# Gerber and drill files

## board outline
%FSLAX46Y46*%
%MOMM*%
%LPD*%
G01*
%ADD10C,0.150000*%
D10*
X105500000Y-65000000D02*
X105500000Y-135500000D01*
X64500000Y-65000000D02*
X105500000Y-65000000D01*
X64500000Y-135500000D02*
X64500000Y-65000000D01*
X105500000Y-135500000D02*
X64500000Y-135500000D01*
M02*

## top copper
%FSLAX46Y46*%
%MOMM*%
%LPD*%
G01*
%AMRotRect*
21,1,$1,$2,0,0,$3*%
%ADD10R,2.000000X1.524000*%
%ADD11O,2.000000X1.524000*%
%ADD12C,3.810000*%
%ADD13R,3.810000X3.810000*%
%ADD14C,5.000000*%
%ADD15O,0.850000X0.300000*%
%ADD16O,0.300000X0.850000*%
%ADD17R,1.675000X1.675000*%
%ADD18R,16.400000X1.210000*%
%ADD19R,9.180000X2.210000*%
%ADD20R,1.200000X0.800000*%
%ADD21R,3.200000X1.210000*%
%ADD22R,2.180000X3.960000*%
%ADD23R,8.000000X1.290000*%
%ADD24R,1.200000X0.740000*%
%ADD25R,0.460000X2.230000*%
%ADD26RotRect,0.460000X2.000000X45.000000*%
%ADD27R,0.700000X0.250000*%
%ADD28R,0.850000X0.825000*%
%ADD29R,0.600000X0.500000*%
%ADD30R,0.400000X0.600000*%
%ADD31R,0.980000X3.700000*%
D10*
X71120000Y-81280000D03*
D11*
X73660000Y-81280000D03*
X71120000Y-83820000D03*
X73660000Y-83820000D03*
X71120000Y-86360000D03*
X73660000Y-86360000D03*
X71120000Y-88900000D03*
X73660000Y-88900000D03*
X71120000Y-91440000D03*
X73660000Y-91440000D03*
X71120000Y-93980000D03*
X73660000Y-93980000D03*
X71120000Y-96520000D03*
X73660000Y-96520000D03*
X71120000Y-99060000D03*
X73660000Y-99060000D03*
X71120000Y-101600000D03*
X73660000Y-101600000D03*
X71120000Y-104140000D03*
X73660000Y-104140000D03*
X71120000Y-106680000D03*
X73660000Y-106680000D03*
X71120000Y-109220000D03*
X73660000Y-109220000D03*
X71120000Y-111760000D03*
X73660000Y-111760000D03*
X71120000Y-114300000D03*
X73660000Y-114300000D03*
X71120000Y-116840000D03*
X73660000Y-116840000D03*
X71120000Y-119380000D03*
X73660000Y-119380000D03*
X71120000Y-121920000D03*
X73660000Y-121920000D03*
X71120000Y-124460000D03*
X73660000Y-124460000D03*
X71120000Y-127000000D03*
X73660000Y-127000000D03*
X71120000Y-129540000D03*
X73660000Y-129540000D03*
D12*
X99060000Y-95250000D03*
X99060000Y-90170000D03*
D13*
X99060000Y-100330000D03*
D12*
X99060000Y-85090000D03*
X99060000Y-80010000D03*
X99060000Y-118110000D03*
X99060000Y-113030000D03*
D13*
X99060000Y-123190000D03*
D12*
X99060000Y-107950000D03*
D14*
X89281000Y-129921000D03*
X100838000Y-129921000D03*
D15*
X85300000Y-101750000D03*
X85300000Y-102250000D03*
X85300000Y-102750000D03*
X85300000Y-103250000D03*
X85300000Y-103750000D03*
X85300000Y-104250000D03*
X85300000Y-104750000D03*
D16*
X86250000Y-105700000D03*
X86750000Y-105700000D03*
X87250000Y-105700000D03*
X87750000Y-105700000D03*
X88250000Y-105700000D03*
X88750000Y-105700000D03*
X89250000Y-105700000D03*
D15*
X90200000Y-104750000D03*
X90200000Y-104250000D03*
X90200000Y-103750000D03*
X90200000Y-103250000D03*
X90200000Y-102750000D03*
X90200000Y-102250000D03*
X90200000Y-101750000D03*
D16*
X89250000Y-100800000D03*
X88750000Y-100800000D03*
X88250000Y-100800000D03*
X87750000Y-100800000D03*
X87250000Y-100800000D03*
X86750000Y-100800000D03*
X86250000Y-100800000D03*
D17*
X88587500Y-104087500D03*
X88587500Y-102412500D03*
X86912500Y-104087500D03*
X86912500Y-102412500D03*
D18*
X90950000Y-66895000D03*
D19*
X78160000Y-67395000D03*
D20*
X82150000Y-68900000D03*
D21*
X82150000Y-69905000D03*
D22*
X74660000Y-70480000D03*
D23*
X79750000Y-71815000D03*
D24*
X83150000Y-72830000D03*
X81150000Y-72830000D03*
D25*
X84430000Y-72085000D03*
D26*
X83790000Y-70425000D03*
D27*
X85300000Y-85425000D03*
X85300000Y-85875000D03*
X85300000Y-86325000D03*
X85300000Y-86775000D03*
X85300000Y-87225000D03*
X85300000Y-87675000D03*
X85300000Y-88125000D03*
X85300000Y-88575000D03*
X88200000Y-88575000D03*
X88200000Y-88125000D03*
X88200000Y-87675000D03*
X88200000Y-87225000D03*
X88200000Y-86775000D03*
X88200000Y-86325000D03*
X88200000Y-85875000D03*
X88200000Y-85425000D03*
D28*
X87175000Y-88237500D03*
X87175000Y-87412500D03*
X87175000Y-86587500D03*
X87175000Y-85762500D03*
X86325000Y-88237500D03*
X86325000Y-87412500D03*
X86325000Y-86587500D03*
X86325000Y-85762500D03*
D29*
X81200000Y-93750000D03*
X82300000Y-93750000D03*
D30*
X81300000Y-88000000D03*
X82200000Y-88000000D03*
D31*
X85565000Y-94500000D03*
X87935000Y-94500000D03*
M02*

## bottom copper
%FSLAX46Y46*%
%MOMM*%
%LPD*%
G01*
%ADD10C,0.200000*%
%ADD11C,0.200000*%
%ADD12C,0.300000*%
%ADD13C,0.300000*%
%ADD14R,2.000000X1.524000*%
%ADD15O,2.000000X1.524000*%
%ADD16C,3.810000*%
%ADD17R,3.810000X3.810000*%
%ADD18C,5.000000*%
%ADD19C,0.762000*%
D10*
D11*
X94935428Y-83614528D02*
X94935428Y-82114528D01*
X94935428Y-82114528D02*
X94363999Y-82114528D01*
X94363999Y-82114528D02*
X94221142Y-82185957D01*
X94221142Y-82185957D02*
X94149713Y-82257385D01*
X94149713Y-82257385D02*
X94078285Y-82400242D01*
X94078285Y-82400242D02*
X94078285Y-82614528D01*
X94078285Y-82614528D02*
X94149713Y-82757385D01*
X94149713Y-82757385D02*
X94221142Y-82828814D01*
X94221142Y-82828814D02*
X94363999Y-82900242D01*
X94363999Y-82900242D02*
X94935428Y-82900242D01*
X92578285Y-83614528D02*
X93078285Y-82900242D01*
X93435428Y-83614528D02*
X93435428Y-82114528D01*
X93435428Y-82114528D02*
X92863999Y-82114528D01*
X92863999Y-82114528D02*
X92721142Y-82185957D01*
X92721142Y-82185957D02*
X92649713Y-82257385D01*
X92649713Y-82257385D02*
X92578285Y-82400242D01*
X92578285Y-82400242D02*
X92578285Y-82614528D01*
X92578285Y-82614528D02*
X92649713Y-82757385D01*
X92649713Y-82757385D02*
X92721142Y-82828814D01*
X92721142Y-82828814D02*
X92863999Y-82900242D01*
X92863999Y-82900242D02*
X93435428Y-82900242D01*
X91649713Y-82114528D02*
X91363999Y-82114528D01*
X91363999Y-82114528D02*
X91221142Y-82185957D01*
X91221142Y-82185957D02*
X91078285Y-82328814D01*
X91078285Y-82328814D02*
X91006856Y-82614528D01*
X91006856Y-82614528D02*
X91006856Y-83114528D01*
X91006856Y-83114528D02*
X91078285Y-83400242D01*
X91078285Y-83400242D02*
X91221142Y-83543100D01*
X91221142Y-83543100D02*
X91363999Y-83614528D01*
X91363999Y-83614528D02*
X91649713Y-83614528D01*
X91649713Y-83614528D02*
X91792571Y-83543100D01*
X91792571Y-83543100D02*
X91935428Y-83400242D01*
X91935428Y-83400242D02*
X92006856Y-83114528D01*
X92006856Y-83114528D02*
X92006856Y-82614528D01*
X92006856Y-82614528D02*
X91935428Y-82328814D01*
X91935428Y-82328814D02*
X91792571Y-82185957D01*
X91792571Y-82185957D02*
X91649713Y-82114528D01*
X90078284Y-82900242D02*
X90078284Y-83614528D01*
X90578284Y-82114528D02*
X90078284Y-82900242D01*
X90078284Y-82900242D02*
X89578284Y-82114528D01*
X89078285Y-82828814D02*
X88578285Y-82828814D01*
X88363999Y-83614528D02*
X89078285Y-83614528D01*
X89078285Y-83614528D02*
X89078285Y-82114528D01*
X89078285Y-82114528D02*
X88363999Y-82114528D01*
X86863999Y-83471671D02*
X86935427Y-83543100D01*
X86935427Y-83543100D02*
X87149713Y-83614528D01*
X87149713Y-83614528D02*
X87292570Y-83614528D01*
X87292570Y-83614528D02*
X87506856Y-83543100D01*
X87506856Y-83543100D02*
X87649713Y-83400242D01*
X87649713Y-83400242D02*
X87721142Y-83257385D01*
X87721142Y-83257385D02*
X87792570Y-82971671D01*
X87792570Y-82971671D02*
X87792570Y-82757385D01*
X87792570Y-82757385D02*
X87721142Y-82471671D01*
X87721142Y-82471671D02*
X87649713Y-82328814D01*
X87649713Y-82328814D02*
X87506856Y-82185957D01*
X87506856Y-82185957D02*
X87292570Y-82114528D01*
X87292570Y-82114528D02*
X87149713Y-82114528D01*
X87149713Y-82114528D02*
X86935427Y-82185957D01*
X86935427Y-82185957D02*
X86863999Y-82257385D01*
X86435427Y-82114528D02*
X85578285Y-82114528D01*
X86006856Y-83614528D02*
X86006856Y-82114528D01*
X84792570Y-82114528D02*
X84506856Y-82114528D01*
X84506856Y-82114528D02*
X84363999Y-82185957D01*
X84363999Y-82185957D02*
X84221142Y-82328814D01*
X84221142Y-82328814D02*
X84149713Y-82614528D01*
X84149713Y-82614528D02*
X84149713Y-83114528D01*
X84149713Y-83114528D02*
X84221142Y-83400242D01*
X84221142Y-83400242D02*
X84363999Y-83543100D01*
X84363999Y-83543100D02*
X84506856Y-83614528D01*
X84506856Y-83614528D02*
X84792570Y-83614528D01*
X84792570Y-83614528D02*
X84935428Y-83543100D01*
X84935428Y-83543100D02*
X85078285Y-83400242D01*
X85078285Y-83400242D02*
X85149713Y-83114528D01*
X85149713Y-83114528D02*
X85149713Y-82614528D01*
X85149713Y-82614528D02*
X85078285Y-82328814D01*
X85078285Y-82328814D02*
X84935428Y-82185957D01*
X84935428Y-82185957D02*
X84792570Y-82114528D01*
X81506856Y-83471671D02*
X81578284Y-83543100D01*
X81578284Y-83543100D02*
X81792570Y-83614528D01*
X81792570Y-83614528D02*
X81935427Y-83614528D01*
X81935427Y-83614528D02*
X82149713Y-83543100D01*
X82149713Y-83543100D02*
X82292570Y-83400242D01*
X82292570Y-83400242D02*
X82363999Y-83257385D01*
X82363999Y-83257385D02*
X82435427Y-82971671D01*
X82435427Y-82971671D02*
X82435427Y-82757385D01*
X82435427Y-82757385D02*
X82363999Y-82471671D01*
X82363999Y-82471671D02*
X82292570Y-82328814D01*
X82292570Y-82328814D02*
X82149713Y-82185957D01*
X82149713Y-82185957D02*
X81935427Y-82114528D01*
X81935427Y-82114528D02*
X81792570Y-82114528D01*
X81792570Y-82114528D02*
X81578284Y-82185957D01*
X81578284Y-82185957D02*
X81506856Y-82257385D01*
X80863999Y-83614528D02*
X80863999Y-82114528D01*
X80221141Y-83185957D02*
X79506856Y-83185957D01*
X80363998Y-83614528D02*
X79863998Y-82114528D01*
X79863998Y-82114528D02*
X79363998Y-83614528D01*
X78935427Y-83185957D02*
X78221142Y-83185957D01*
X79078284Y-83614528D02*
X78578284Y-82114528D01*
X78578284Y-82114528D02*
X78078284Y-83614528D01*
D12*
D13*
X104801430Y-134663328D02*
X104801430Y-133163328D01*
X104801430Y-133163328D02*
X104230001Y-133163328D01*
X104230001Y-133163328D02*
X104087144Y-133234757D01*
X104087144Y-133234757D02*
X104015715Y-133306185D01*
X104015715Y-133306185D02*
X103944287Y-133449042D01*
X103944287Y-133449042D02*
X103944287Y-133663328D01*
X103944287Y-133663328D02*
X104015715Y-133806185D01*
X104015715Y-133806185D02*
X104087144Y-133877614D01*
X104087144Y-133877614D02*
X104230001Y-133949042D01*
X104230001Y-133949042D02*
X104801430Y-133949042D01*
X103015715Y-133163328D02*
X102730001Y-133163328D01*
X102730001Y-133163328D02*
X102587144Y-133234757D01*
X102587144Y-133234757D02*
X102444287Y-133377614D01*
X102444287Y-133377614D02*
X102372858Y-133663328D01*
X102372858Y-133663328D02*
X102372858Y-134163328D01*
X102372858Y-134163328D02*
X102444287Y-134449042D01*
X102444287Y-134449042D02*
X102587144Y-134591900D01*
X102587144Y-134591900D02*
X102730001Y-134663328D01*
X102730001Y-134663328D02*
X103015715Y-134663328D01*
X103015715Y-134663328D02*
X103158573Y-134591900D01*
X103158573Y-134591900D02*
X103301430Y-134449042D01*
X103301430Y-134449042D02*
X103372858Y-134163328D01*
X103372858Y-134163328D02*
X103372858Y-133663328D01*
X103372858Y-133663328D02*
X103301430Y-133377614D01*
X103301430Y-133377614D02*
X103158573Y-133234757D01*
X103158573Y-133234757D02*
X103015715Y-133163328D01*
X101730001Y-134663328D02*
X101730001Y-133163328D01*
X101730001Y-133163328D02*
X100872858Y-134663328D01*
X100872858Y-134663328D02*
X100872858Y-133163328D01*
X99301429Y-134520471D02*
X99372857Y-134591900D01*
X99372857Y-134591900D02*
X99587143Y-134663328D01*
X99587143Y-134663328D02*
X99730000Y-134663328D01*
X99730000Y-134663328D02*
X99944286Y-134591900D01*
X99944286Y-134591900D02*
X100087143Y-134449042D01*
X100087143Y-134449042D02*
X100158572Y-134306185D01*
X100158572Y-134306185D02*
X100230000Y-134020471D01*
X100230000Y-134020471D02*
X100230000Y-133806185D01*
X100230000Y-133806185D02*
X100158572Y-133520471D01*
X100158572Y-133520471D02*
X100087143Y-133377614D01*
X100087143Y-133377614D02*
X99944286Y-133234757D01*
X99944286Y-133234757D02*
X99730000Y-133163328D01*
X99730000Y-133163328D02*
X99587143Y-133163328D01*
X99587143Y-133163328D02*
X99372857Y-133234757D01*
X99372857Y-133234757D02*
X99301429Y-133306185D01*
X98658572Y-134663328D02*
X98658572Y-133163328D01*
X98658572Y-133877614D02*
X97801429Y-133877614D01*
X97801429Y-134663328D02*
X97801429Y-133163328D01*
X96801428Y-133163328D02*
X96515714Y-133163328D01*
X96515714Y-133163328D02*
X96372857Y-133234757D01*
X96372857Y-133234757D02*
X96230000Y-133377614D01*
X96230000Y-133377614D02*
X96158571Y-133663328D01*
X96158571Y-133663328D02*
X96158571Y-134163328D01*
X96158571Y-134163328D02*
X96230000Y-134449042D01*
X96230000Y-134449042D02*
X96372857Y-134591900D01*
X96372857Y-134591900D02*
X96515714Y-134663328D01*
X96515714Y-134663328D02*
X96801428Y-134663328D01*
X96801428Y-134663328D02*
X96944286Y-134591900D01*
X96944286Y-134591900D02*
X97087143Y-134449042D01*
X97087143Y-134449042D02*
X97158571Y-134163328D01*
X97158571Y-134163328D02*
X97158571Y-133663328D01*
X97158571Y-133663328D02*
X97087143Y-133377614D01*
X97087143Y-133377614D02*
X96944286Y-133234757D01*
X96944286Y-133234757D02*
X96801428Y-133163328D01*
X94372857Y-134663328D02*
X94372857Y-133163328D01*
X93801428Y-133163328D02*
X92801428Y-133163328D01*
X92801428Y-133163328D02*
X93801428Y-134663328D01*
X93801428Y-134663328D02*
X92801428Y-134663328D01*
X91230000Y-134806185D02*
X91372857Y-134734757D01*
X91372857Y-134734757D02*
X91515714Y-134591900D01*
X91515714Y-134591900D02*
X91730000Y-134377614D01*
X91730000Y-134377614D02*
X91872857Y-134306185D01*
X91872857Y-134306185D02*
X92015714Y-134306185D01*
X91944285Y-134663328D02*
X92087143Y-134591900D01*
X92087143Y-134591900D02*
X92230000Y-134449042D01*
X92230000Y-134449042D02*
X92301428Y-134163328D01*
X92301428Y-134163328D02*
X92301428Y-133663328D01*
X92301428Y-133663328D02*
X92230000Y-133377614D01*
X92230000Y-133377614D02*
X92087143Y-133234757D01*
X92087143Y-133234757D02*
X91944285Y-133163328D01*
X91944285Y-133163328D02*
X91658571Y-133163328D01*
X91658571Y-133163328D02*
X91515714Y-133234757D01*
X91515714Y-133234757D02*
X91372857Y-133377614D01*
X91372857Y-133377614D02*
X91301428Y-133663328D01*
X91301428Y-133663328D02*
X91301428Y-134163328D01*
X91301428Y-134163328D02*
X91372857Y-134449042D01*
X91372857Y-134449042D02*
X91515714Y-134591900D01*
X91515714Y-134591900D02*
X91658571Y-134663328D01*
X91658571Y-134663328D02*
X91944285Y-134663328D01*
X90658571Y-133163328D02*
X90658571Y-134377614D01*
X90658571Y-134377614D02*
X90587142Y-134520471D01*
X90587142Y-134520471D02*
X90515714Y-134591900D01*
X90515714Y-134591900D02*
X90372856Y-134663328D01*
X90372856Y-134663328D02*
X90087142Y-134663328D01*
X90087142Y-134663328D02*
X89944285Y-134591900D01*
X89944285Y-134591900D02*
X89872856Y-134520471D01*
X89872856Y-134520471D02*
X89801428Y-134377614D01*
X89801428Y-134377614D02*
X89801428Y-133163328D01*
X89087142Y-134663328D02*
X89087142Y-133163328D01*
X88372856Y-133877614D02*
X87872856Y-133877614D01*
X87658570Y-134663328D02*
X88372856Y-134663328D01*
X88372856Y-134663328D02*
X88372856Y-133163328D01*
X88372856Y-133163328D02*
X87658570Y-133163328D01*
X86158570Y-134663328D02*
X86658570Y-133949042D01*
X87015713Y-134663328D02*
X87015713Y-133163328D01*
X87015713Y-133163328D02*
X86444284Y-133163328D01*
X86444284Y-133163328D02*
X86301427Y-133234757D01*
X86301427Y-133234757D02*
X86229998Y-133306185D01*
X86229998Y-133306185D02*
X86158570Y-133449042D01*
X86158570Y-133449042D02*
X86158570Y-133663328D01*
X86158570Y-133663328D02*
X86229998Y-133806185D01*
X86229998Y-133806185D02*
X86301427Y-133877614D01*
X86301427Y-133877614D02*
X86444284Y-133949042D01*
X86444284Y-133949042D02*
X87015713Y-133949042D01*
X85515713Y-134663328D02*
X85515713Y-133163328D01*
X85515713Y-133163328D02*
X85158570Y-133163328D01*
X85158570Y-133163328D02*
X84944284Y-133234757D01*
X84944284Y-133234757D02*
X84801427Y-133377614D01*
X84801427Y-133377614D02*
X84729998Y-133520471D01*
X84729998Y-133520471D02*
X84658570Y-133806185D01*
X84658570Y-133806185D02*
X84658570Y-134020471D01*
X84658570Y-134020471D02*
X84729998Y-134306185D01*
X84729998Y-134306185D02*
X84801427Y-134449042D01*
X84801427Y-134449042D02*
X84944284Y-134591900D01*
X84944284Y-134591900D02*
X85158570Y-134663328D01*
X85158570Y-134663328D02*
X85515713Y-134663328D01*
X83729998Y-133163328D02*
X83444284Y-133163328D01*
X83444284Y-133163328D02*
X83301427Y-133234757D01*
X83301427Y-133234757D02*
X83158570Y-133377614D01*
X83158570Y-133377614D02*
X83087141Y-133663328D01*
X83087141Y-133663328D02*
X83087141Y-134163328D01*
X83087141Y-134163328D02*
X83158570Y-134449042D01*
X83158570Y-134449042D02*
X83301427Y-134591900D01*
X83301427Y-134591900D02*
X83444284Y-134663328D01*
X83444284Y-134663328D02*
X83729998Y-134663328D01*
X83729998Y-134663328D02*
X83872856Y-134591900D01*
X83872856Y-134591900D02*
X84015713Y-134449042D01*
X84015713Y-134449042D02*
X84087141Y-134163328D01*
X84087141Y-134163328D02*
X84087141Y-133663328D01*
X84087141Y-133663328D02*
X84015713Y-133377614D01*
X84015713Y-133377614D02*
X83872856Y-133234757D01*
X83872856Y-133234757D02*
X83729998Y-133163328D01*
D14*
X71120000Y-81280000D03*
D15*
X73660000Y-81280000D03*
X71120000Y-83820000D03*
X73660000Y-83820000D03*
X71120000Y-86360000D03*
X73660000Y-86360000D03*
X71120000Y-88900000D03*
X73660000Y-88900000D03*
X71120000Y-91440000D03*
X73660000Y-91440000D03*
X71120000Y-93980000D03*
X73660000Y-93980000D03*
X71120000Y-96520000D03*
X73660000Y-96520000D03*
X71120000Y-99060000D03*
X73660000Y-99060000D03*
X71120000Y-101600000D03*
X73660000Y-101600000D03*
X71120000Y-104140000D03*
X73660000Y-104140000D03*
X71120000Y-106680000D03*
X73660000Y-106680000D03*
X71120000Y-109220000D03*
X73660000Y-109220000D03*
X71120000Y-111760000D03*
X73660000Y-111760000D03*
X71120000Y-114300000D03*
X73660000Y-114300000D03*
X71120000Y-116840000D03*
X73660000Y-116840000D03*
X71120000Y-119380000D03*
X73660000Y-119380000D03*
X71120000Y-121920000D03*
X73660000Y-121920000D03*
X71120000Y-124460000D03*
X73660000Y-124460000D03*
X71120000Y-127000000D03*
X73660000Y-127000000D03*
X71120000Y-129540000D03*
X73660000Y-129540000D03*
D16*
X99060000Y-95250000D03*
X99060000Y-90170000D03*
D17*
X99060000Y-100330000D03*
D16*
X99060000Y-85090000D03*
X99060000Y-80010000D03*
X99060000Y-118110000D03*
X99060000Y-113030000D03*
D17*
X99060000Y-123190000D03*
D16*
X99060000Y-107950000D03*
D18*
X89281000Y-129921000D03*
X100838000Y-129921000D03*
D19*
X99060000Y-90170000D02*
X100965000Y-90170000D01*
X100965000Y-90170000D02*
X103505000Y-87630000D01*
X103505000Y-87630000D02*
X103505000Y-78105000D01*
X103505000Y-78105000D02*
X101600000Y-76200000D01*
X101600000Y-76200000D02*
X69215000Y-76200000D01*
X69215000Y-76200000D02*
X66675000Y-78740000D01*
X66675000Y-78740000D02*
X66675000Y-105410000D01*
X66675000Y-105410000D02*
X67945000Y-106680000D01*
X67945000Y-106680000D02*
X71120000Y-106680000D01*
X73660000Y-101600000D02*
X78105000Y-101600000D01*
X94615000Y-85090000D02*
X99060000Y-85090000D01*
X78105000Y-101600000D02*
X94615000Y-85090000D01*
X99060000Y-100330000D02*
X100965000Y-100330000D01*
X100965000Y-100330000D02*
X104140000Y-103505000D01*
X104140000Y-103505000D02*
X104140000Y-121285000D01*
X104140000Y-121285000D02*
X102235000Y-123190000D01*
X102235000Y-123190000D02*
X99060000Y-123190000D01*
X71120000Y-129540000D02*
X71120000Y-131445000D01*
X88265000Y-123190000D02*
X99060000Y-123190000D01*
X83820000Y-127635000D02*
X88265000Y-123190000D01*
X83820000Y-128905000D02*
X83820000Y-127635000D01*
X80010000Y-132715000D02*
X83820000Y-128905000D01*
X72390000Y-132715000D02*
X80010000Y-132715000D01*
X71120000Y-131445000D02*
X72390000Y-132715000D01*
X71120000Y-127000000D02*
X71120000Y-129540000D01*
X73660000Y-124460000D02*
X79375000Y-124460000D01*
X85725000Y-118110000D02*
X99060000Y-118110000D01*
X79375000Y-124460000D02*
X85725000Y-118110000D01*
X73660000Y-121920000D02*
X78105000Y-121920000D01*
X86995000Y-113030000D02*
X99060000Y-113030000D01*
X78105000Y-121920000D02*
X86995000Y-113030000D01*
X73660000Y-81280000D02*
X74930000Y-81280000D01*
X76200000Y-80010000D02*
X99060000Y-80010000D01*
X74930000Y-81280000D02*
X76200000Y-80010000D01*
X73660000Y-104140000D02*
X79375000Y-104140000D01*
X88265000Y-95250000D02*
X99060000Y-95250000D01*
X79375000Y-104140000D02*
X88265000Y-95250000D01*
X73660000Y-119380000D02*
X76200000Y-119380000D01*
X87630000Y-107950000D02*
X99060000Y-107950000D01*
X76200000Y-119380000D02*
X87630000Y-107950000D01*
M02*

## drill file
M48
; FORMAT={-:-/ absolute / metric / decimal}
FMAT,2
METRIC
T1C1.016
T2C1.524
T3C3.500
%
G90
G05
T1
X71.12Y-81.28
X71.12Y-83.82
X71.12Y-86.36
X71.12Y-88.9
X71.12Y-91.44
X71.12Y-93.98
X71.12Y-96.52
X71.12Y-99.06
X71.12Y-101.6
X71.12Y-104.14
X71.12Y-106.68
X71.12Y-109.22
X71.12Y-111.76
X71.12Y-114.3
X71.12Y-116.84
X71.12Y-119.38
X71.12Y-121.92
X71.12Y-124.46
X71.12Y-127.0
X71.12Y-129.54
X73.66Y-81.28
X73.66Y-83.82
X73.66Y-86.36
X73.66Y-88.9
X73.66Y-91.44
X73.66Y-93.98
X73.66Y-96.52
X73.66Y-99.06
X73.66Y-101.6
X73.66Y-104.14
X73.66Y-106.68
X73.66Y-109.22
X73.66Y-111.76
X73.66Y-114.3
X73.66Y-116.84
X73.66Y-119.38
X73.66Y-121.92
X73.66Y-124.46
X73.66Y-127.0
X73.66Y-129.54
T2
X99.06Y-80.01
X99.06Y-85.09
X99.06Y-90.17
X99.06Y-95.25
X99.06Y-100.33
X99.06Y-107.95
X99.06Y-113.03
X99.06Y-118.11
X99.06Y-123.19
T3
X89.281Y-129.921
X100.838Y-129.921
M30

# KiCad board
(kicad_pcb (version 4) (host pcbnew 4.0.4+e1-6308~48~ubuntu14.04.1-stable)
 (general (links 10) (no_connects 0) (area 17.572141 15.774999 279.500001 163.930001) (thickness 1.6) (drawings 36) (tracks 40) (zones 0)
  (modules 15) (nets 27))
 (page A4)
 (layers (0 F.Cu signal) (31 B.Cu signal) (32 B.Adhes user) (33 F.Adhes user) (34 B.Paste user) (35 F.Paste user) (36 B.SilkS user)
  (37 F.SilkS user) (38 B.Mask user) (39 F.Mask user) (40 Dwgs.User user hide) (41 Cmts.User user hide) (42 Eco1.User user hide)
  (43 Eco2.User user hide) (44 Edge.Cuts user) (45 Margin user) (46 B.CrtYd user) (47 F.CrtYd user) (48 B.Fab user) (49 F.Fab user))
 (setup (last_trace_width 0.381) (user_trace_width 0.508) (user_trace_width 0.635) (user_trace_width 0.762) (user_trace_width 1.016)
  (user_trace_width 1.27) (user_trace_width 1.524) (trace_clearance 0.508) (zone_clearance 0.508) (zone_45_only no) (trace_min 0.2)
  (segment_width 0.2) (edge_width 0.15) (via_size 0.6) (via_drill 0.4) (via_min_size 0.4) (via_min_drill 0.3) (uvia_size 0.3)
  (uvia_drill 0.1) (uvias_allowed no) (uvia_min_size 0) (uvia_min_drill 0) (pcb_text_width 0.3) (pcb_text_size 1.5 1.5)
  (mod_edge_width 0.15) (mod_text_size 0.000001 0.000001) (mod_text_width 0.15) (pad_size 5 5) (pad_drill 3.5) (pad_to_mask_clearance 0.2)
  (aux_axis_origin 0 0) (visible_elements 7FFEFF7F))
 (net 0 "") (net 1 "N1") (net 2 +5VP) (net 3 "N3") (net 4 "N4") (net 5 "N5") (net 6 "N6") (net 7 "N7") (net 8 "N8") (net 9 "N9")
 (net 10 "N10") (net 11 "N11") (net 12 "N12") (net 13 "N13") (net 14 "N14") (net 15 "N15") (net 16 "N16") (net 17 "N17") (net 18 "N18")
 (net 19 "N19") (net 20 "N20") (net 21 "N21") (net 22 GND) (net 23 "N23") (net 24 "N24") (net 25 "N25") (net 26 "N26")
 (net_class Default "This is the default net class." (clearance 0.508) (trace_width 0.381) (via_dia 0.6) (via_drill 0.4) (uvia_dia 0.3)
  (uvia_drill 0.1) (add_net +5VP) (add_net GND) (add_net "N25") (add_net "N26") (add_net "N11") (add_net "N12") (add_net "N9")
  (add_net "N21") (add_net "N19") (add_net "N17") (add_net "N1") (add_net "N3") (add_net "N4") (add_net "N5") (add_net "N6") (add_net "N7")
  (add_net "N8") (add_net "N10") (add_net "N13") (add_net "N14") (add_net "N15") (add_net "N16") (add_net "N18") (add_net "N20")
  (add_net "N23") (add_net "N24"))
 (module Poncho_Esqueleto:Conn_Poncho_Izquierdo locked (layer F.Cu) (at 71.12 81.28)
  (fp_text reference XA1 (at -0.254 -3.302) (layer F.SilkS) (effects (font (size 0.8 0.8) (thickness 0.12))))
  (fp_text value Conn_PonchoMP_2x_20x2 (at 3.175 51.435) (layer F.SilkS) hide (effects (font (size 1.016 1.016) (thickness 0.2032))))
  (pad 41 thru_hole rect (at 0 0 270) (size 1.524 2) (drill 1.016) (layers *.Cu *.Mask F.SilkS) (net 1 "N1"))
  (pad 42 thru_hole oval (at 2.54 0 270) (size 1.524 2) (drill 1.016) (layers *.Cu *.Mask F.SilkS) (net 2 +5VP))
  (pad 43 thru_hole oval (at 0 2.54 270) (size 1.524 2) (drill 1.016) (layers *.Cu *.Mask F.SilkS) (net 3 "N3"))
  (pad 44 thru_hole oval (at 2.54 2.54 270) (size 1.524 2) (drill 1.016) (layers *.Cu *.Mask F.SilkS))
  (pad 45 thru_hole oval (at 0 5.08 270) (size 1.524 2) (drill 1.016) (layers *.Cu *.Mask F.SilkS) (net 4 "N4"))
  (pad 46 thru_hole oval (at 2.54 5.08 270) (size 1.524 2) (drill 1.016) (layers *.Cu *.Mask F.SilkS))
  (pad 47 thru_hole oval (at 0 7.62 270) (size 1.524 2) (drill 1.016) (layers *.Cu *.Mask F.SilkS) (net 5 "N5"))
  (pad 48 thru_hole oval (at 2.54 7.62 270) (size 1.524 2) (drill 1.016) (layers *.Cu *.Mask F.SilkS))
  (pad 49 thru_hole oval (at 0 10.16 270) (size 1.524 2) (drill 1.016) (layers *.Cu *.Mask F.SilkS))
  (pad 50 thru_hole oval (at 2.54 10.16 270) (size 1.524 2) (drill 1.016) (layers *.Cu *.Mask F.SilkS))
  (pad 51 thru_hole oval (at 0 12.7 270) (size 1.524 2) (drill 1.016) (layers *.Cu *.Mask F.SilkS) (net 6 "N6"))
  (pad 52 thru_hole oval (at 2.54 12.7 270) (size 1.524 2) (drill 1.016) (layers *.Cu *.Mask F.SilkS))
  (pad 53 thru_hole oval (at 0 15.24 270) (size 1.524 2) (drill 1.016) (layers *.Cu *.Mask F.SilkS) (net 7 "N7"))
  (pad 54 thru_hole oval (at 2.54 15.24 270) (size 1.524 2) (drill 1.016) (layers *.Cu *.Mask F.SilkS))
  (pad 55 thru_hole oval (at 0 17.78 270) (size 1.524 2) (drill 1.016) (layers *.Cu *.Mask F.SilkS))
  (pad 56 thru_hole oval (at 2.54 17.78 270) (size 1.524 2) (drill 1.016) (layers *.Cu *.Mask F.SilkS))
  (pad 57 thru_hole oval (at 0 20.32 270) (size 1.524 2) (drill 1.016) (layers *.Cu *.Mask F.SilkS) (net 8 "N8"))
  (pad 58 thru_hole oval (at 2.54 20.32 270) (size 1.524 2) (drill 1.016) (layers *.Cu *.Mask F.SilkS) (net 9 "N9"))
  (pad 59 thru_hole oval (at 0 22.86 270) (size 1.524 2) (drill 1.016) (layers *.Cu *.Mask F.SilkS) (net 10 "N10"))
  (pad 60 thru_hole oval (at 2.54 22.86 270) (size 1.524 2) (drill 1.016) (layers *.Cu *.Mask F.SilkS) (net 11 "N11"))
  (pad 61 thru_hole oval (at 0 25.4 270) (size 1.524 2) (drill 1.016) (layers *.Cu *.Mask F.SilkS) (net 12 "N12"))
  (pad 62 thru_hole oval (at 2.54 25.4 270) (size 1.524 2) (drill 1.016) (layers *.Cu *.Mask F.SilkS))
  (pad 63 thru_hole oval (at 0 27.94 270) (size 1.524 2) (drill 1.016) (layers *.Cu *.Mask F.SilkS))
  (pad 64 thru_hole oval (at 2.54 27.94 270) (size 1.524 2) (drill 1.016) (layers *.Cu *.Mask F.SilkS))
  (pad 65 thru_hole oval (at 0 30.48 270) (size 1.524 2) (drill 1.016) (layers *.Cu *.Mask F.SilkS) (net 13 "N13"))
  (pad 66 thru_hole oval (at 2.54 30.48 270) (size 1.524 2) (drill 1.016) (layers *.Cu *.Mask F.SilkS))
  (pad 67 thru_hole oval (at 0 33.02 270) (size 1.524 2) (drill 1.016) (layers *.Cu *.Mask F.SilkS) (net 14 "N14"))
  (pad 68 thru_hole oval (at 2.54 33.02 270) (size 1.524 2) (drill 1.016) (layers *.Cu *.Mask F.SilkS))
  (pad 69 thru_hole oval (at 0 35.56 270) (size 1.524 2) (drill 1.016) (layers *.Cu *.Mask F.SilkS) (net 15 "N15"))
  (pad 70 thru_hole oval (at 2.54 35.56 270) (size 1.524 2) (drill 1.016) (layers *.Cu *.Mask F.SilkS))
  (pad 71 thru_hole oval (at 0 38.1 270) (size 1.524 2) (drill 1.016) (layers *.Cu *.Mask F.SilkS) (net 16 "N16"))
  (pad 72 thru_hole oval (at 2.54 38.1 270) (size 1.524 2) (drill 1.016) (layers *.Cu *.Mask F.SilkS) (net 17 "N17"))
  (pad 73 thru_hole oval (at 0 40.64 270) (size 1.524 2) (drill 1.016) (layers *.Cu *.Mask F.SilkS) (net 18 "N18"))
  (pad 74 thru_hole oval (at 2.54 40.64 270) (size 1.524 2) (drill 1.016) (layers *.Cu *.Mask F.SilkS) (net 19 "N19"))
  (pad 75 thru_hole oval (at 0 43.18 270) (size 1.524 2) (drill 1.016) (layers *.Cu *.Mask F.SilkS) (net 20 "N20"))
  (pad 76 thru_hole oval (at 2.54 43.18 270) (size 1.524 2) (drill 1.016) (layers *.Cu *.Mask F.SilkS) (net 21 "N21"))
  (pad 77 thru_hole oval (at 0 45.72 270) (size 1.524 2) (drill 1.016) (layers *.Cu *.Mask F.SilkS) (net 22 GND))
  (pad 78 thru_hole oval (at 2.54 45.72 270) (size 1.524 2) (drill 1.016) (layers *.Cu *.Mask F.SilkS) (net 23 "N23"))
  (pad 79 thru_hole oval (at 0 48.26 270) (size 1.524 2) (drill 1.016) (layers *.Cu *.Mask F.SilkS) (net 22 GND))
  (pad 80 thru_hole oval (at 2.54 48.26 270) (size 1.524 2) (drill 1.016) (layers *.Cu *.Mask F.SilkS) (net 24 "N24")))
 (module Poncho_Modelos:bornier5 (layer F.Cu) (at 99.06 90.17 90)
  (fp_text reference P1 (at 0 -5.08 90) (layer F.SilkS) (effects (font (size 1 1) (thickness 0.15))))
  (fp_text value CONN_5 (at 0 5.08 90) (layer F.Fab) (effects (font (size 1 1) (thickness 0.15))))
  (pad 2 thru_hole circle (at -5.08 0 90) (size 3.81 3.81) (drill 1.524) (layers *.Cu *.Mask F.SilkS) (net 11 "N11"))
  (pad 3 thru_hole circle (at 0 0 90) (size 3.81 3.81) (drill 1.524) (layers *.Cu *.Mask F.SilkS) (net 12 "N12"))
  (pad 1 thru_hole rect (at -10.16 0 90) (size 3.81 3.81) (drill 1.524) (layers *.Cu *.Mask F.SilkS) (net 22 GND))
  (pad 4 thru_hole circle (at 5.08 0 90) (size 3.81 3.81) (drill 1.524) (layers *.Cu *.Mask F.SilkS) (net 9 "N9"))
  (pad 5 thru_hole circle (at 10.16 0 90) (size 3.81 3.81) (drill 1.524) (layers *.Cu *.Mask F.SilkS) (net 2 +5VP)))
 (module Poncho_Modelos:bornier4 (layer F.Cu) (at 99.06 115.57 90)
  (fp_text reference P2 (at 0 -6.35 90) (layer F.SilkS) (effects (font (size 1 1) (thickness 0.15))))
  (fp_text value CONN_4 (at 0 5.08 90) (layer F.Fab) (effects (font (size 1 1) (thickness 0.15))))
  (pad 2 thru_hole circle (at -2.54 0 90) (size 3.81 3.81) (drill 1.524) (layers *.Cu *.Mask F.SilkS) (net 21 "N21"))
  (pad 3 thru_hole circle (at 2.54 0 90) (size 3.81 3.81) (drill 1.524) (layers *.Cu *.Mask F.SilkS) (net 19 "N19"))
  (pad 1 thru_hole rect (at -7.62 0 90) (size 3.81 3.81) (drill 1.524) (layers *.Cu *.Mask F.SilkS) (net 22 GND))
  (pad 4 thru_hole circle (at 7.62 0 90) (size 3.81 3.81) (drill 1.524) (layers *.Cu *.Mask F.SilkS) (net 17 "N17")))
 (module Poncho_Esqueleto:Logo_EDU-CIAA (layer F.Cu) (at 87.63 116.205)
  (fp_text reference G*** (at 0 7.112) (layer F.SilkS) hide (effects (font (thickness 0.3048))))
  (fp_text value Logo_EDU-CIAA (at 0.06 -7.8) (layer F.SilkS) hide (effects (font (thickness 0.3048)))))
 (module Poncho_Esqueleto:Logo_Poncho (layer F.Cu) (at 100.75 71.25)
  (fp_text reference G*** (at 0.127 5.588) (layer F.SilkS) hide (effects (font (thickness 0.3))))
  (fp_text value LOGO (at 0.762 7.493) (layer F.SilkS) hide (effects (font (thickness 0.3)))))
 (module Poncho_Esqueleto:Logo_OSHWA (layer F.Cu) (at 68.75 70.5)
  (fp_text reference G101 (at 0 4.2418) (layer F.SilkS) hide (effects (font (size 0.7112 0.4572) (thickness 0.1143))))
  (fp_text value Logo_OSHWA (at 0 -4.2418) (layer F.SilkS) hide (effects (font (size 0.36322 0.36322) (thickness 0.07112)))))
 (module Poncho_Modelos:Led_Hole (layer F.Cu) (at 89.281 129.921)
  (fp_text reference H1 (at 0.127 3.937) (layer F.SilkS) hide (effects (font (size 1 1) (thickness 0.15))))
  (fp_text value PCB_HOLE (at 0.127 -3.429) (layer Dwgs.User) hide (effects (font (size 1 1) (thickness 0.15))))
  (pad 1 thru_hole circle (at 0 0) (size 5 5) (drill 3.5) (layers *.Cu *.Mask F.SilkS) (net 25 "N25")))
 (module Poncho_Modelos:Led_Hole (layer F.Cu) (at 100.838 129.921)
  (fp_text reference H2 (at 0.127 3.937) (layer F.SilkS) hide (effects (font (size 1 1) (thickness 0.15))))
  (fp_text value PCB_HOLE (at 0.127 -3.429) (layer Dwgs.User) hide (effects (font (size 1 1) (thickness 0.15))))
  (pad 1 thru_hole circle (at 0 0) (size 5 5) (drill 3.5) (layers *.Cu *.Mask F.SilkS) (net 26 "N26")))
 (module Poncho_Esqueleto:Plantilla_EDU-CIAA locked (layer F.Cu) (at 142.24 81.28)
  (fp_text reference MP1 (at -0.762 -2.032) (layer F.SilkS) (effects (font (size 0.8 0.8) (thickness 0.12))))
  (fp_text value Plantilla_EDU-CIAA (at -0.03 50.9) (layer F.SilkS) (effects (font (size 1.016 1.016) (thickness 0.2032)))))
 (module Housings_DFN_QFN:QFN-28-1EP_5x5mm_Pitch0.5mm (layer F.Cu) (at 87.75 103.25)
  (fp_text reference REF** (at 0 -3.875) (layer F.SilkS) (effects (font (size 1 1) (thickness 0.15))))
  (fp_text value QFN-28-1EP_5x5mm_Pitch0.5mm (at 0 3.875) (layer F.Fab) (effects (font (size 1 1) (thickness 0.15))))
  (pad 1 smd oval (at -2.45 -1.5) (size 0.85 0.3) (layers F.Cu F.Paste F.Mask))
  (pad 2 smd oval (at -2.45 -1) (size 0.85 0.3) (layers F.Cu F.Paste F.Mask))
  (pad 3 smd oval (at -2.45 -0.5) (size 0.85 0.3) (layers F.Cu F.Paste F.Mask))
  (pad 4 smd oval (at -2.45 0) (size 0.85 0.3) (layers F.Cu F.Paste F.Mask))
  (pad 5 smd oval (at -2.45 0.5) (size 0.85 0.3) (layers F.Cu F.Paste F.Mask))
  (pad 6 smd oval (at -2.45 1) (size 0.85 0.3) (layers F.Cu F.Paste F.Mask))
  (pad 7 smd oval (at -2.45 1.5) (size 0.85 0.3) (layers F.Cu F.Paste F.Mask))
  (pad 8 smd oval (at -1.5 2.45 90) (size 0.85 0.3) (layers F.Cu F.Paste F.Mask))
  (pad 9 smd oval (at -1 2.45 90) (size 0.85 0.3) (layers F.Cu F.Paste F.Mask))
  (pad 10 smd oval (at -0.5 2.45 90) (size 0.85 0.3) (layers F.Cu F.Paste F.Mask))
  (pad 11 smd oval (at 0 2.45 90) (size 0.85 0.3) (layers F.Cu F.Paste F.Mask))
  (pad 12 smd oval (at 0.5 2.45 90) (size 0.85 0.3) (layers F.Cu F.Paste F.Mask))
  (pad 13 smd oval (at 1 2.45 90) (size 0.85 0.3) (layers F.Cu F.Paste F.Mask))
  (pad 14 smd oval (at 1.5 2.45 90) (size 0.85 0.3) (layers F.Cu F.Paste F.Mask))
  (pad 15 smd oval (at 2.45 1.5) (size 0.85 0.3) (layers F.Cu F.Paste F.Mask))
  (pad 16 smd oval (at 2.45 1) (size 0.85 0.3) (layers F.Cu F.Paste F.Mask))
  (pad 17 smd oval (at 2.45 0.5) (size 0.85 0.3) (layers F.Cu F.Paste F.Mask))
  (pad 18 smd oval (at 2.45 0) (size 0.85 0.3) (layers F.Cu F.Paste F.Mask))
  (pad 19 smd oval (at 2.45 -0.5) (size 0.85 0.3) (layers F.Cu F.Paste F.Mask))
  (pad 20 smd oval (at 2.45 -1) (size 0.85 0.3) (layers F.Cu F.Paste F.Mask))
  (pad 21 smd oval (at 2.45 -1.5) (size 0.85 0.3) (layers F.Cu F.Paste F.Mask))
  (pad 22 smd oval (at 1.5 -2.45 90) (size 0.85 0.3) (layers F.Cu F.Paste F.Mask))
  (pad 23 smd oval (at 1 -2.45 90) (size 0.85 0.3) (layers F.Cu F.Paste F.Mask))
  (pad 24 smd oval (at 0.5 -2.45 90) (size 0.85 0.3) (layers F.Cu F.Paste F.Mask))
  (pad 25 smd oval (at 0 -2.45 90) (size 0.85 0.3) (layers F.Cu F.Paste F.Mask))
  (pad 26 smd oval (at -0.5 -2.45 90) (size 0.85 0.3) (layers F.Cu F.Paste F.Mask))
  (pad 27 smd oval (at -1 -2.45 90) (size 0.85 0.3) (layers F.Cu F.Paste F.Mask))
  (pad 28 smd oval (at -1.5 -2.45 90) (size 0.85 0.3) (layers F.Cu F.Paste F.Mask))
  (pad 29 smd rect (at 0.8375 0.8375) (size 1.675 1.675) (layers F.Cu F.Paste F.Mask) (solder_paste_margin_ratio -0.2))
  (pad 29 smd rect (at 0.8375 -0.8375) (size 1.675 1.675) (layers F.Cu F.Paste F.Mask) (solder_paste_margin_ratio -0.2))
  (pad 29 smd rect (at -0.8375 0.8375) (size 1.675 1.675) (layers F.Cu F.Paste F.Mask) (solder_paste_margin_ratio -0.2))
  (pad 29 smd rect (at -0.8375 -0.8375) (size 1.675 1.675) (layers F.Cu F.Paste F.Mask) (solder_paste_margin_ratio -0.2)))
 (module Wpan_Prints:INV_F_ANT (layer F.Cu) (at 82.75 67.5)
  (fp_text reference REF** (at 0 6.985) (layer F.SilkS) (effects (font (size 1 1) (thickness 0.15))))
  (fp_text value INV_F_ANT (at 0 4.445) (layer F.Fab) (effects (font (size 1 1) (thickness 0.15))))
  (pad "" smd rect (at 8.2 -0.605) (size 16.4 1.21) (layers F.Cu F.Paste))
  (pad "" smd rect (at -4.59 -0.105) (size 9.18 2.21) (layers F.Cu F.Paste))
  (pad "" smd rect (at -0.6 1.4) (size 1.2 0.8) (layers F.Cu F.Paste))
  (pad "" smd rect (at -0.6 2.405) (size 3.2 1.21) (layers F.Cu F.Paste))
  (pad "" smd rect (at -8.09 2.98) (size 2.18 3.96) (layers F.Cu F.Paste))
  (pad "" smd rect (at -3 4.315) (size 8 1.29) (layers F.Cu F.Paste))
  (pad 2 smd rect (at 0.4 5.33) (size 1.2 0.74) (layers F.Cu F.Paste) (zone_connect 2))
  (pad 3 smd rect (at -1.6 5.33) (size 1.2 0.74) (layers F.Cu F.Paste) (zone_connect 2))
  (pad 1 smd rect (at 1.68 4.585) (size 0.46 2.23) (layers F.Cu F.Paste))
  (pad "" smd rect (at 1.04 2.925 45) (size 0.46 2) (layers F.Cu F.Paste)))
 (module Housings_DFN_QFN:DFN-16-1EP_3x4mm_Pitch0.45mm (layer F.Cu) (at 86.75 87)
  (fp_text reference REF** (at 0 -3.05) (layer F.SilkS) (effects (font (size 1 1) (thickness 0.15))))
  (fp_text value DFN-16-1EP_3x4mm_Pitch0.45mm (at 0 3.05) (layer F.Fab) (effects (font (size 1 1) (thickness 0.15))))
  (pad 1 smd rect (at -1.45 -1.575) (size 0.7 0.25) (layers F.Cu F.Paste F.Mask))
  (pad 2 smd rect (at -1.45 -1.125) (size 0.7 0.25) (layers F.Cu F.Paste F.Mask))
  (pad 3 smd rect (at -1.45 -0.675) (size 0.7 0.25) (layers F.Cu F.Paste F.Mask))
  (pad 4 smd rect (at -1.45 -0.225) (size 0.7 0.25) (layers F.Cu F.Paste F.Mask))
  (pad 5 smd rect (at -1.45 0.225) (size 0.7 0.25) (layers F.Cu F.Paste F.Mask))
  (pad 6 smd rect (at -1.45 0.675) (size 0.7 0.25) (layers F.Cu F.Paste F.Mask))
  (pad 7 smd rect (at -1.45 1.125) (size 0.7 0.25) (layers F.Cu F.Paste F.Mask))
  (pad 8 smd rect (at -1.45 1.575) (size 0.7 0.25) (layers F.Cu F.Paste F.Mask))
  (pad 9 smd rect (at 1.45 1.575) (size 0.7 0.25) (layers F.Cu F.Paste F.Mask))
  (pad 10 smd rect (at 1.45 1.125) (size 0.7 0.25) (layers F.Cu F.Paste F.Mask))
  (pad 11 smd rect (at 1.45 0.675) (size 0.7 0.25) (layers F.Cu F.Paste F.Mask))
  (pad 12 smd rect (at 1.45 0.225) (size 0.7 0.25) (layers F.Cu F.Paste F.Mask))
  (pad 13 smd rect (at 1.45 -0.225) (size 0.7 0.25) (layers F.Cu F.Paste F.Mask))
  (pad 14 smd rect (at 1.45 -0.675) (size 0.7 0.25) (layers F.Cu F.Paste F.Mask))
  (pad 15 smd rect (at 1.45 -1.125) (size 0.7 0.25) (layers F.Cu F.Paste F.Mask))
  (pad 16 smd rect (at 1.45 -1.575) (size 0.7 0.25) (layers F.Cu F.Paste F.Mask))
  (pad 17 smd rect (at 0.425 1.2375) (size 0.85 0.825) (layers F.Cu F.Paste F.Mask) (solder_paste_margin_ratio -0.2))
  (pad 17 smd rect (at 0.425 0.4125) (size 0.85 0.825) (layers F.Cu F.Paste F.Mask) (solder_paste_margin_ratio -0.2))
  (pad 17 smd rect (at 0.425 -0.4125) (size 0.85 0.825) (layers F.Cu F.Paste F.Mask) (solder_paste_margin_ratio -0.2))
  (pad 17 smd rect (at 0.425 -1.2375) (size 0.85 0.825) (layers F.Cu F.Paste F.Mask) (solder_paste_margin_ratio -0.2))
  (pad 17 smd rect (at -0.425 1.2375) (size 0.85 0.825) (layers F.Cu F.Paste F.Mask) (solder_paste_margin_ratio -0.2))
  (pad 17 smd rect (at -0.425 0.4125) (size 0.85 0.825) (layers F.Cu F.Paste F.Mask) (solder_paste_margin_ratio -0.2))
  (pad 17 smd rect (at -0.425 -0.4125) (size 0.85 0.825) (layers F.Cu F.Paste F.Mask) (solder_paste_margin_ratio -0.2))
  (pad 17 smd rect (at -0.425 -1.2375) (size 0.85 0.825) (layers F.Cu F.Paste F.Mask) (solder_paste_margin_ratio -0.2)))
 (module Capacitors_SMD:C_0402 (layer F.Cu) (at 81.75 93.75)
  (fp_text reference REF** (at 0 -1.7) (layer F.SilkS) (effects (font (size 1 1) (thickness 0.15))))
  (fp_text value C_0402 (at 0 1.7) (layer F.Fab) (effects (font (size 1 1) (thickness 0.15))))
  (pad 1 smd rect (at -0.55 0) (size 0.6 0.5) (layers F.Cu F.Paste F.Mask))
  (pad 2 smd rect (at 0.55 0) (size 0.6 0.5) (layers F.Cu F.Paste F.Mask)))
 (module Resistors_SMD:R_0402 (layer F.Cu) (at 81.75 88)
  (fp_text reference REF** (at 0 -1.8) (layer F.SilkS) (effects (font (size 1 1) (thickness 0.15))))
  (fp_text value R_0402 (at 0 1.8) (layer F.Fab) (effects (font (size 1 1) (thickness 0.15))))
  (pad 1 smd rect (at -0.45 0) (size 0.4 0.6) (layers F.Cu F.Paste F.Mask))
  (pad 2 smd rect (at 0.45 0) (size 0.4 0.6) (layers F.Cu F.Paste F.Mask)))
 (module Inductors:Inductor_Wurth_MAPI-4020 (layer F.Cu) (at 86.75 94.5)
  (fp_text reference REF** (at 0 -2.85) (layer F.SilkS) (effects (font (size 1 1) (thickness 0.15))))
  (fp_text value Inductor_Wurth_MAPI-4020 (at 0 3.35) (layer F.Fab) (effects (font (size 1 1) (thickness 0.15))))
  (pad 1 smd rect (at -1.185 0) (size 0.98 3.7) (layers F.Cu F.Paste F.Mask))
  (pad 2 smd rect (at 1.185 0) (size 0.98 3.7) (layers F.Cu F.Paste F.Mask)))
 (gr_line (start 105.5 65) (end 105.5 135.5) (angle 90) (layer Edge.Cuts) (width 0.15))
 (gr_line (start 64.5 65) (end 105.5 65) (angle 90) (layer Edge.Cuts) (width 0.15))
 (gr_line (start 64.5 135.5) (end 64.5 65) (angle 90) (layer Edge.Cuts) (width 0.15))
 (gr_line (start 105.5 135.5) (end 64.5 135.5) (angle 90) (layer Edge.Cuts) (width 0.15))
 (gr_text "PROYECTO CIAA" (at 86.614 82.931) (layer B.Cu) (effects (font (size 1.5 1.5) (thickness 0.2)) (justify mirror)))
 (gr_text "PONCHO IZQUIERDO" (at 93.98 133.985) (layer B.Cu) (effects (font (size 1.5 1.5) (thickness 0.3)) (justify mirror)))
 (segment (start 99.06 90.17) (end 100.965 90.17) (width 0.762) (layer B.Cu) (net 12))
 (segment (start 100.965 90.17) (end 103.505 87.63) (width 0.762) (layer B.Cu) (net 12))
 (segment (start 103.505 87.63) (end 103.505 78.105) (width 0.762) (layer B.Cu) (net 12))
 (segment (start 103.505 78.105) (end 101.6 76.2) (width 0.762) (layer B.Cu) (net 12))
 (segment (start 101.6 76.2) (end 69.215 76.2) (width 0.762) (layer B.Cu) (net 12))
 (segment (start 69.215 76.2) (end 66.675 78.74) (width 0.762) (layer B.Cu) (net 12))
 (segment (start 66.675 78.74) (end 66.675 105.41) (width 0.762) (layer B.Cu) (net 12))
 (segment (start 66.675 105.41) (end 67.945 106.68) (width 0.762) (layer B.Cu) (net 12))
 (segment (start 67.945 106.68) (end 71.12 106.68) (width 0.762) (layer B.Cu) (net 12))
 (segment (start 73.66 101.6) (end 78.105 101.6) (width 0.762) (layer B.Cu) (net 9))
 (segment (start 94.615 85.09) (end 99.06 85.09) (width 0.762) (layer B.Cu) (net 9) (status 20))
 (segment (start 78.105 101.6) (end 94.615 85.09) (width 0.762) (layer B.Cu) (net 9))
 (segment (start 99.06 100.33) (end 100.965 100.33) (width 0.762) (layer B.Cu) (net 22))
 (segment (start 100.965 100.33) (end 104.14 103.505) (width 0.762) (layer B.Cu) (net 22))
 (segment (start 104.14 103.505) (end 104.14 121.285) (width 0.762) (layer B.Cu) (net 22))
 (segment (start 104.14 121.285) (end 102.235 123.19) (width 0.762) (layer B.Cu) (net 22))
 (segment (start 102.235 123.19) (end 99.06 123.19) (width 0.762) (layer B.Cu) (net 22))
 (segment (start 71.12 129.54) (end 71.12 131.445) (width 0.762) (layer B.Cu) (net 22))
 (segment (start 88.265 123.19) (end 99.06 123.19) (width 0.762) (layer B.Cu) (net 22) (status 20))
 (segment (start 83.82 127.635) (end 88.265 123.19) (width 0.762) (layer B.Cu) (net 22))
 (segment (start 83.82 128.905) (end 83.82 127.635) (width 0.762) (layer B.Cu) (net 22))
 (segment (start 80.01 132.715) (end 83.82 128.905) (width 0.762) (layer B.Cu) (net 22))
 (segment (start 72.39 132.715) (end 80.01 132.715) (width 0.762) (layer B.Cu) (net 22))
 (segment (start 71.12 131.445) (end 72.39 132.715) (width 0.762) (layer B.Cu) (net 22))
 (segment (start 71.12 127) (end 71.12 129.54) (width 0.762) (layer B.Cu) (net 22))
 (segment (start 73.66 124.46) (end 79.375 124.46) (width 0.762) (layer B.Cu) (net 21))
 (segment (start 85.725 118.11) (end 99.06 118.11) (width 0.762) (layer B.Cu) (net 21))
 (segment (start 79.375 124.46) (end 85.725 118.11) (width 0.762) (layer B.Cu) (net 21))
 (segment (start 73.66 121.92) (end 78.105 121.92) (width 0.762) (layer B.Cu) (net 19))
 (segment (start 86.995 113.03) (end 99.06 113.03) (width 0.762) (layer B.Cu) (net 19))
 (segment (start 78.105 121.92) (end 86.995 113.03) (width 0.762) (layer B.Cu) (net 19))
 (segment (start 73.66 81.28) (end 74.93 81.28) (width 0.762) (layer B.Cu) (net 2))
 (segment (start 76.2 80.01) (end 99.06 80.01) (width 0.762) (layer B.Cu) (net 2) (status 20))
 (segment (start 74.93 81.28) (end 76.2 80.01) (width 0.762) (layer B.Cu) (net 2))
 (segment (start 73.66 104.14) (end 79.375 104.14) (width 0.762) (layer B.Cu) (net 11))
 (segment (start 88.265 95.25) (end 99.06 95.25) (width 0.762) (layer B.Cu) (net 11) (status 20))
 (segment (start 79.375 104.14) (end 88.265 95.25) (width 0.762) (layer B.Cu) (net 11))
 (segment (start 73.66 119.38) (end 76.2 119.38) (width 0.762) (layer B.Cu) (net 17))
 (segment (start 87.63 107.95) (end 99.06 107.95) (width 0.762) (layer B.Cu) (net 17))
 (segment (start 76.2 119.38) (end 87.63 107.95) (width 0.762) (layer B.Cu) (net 17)))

